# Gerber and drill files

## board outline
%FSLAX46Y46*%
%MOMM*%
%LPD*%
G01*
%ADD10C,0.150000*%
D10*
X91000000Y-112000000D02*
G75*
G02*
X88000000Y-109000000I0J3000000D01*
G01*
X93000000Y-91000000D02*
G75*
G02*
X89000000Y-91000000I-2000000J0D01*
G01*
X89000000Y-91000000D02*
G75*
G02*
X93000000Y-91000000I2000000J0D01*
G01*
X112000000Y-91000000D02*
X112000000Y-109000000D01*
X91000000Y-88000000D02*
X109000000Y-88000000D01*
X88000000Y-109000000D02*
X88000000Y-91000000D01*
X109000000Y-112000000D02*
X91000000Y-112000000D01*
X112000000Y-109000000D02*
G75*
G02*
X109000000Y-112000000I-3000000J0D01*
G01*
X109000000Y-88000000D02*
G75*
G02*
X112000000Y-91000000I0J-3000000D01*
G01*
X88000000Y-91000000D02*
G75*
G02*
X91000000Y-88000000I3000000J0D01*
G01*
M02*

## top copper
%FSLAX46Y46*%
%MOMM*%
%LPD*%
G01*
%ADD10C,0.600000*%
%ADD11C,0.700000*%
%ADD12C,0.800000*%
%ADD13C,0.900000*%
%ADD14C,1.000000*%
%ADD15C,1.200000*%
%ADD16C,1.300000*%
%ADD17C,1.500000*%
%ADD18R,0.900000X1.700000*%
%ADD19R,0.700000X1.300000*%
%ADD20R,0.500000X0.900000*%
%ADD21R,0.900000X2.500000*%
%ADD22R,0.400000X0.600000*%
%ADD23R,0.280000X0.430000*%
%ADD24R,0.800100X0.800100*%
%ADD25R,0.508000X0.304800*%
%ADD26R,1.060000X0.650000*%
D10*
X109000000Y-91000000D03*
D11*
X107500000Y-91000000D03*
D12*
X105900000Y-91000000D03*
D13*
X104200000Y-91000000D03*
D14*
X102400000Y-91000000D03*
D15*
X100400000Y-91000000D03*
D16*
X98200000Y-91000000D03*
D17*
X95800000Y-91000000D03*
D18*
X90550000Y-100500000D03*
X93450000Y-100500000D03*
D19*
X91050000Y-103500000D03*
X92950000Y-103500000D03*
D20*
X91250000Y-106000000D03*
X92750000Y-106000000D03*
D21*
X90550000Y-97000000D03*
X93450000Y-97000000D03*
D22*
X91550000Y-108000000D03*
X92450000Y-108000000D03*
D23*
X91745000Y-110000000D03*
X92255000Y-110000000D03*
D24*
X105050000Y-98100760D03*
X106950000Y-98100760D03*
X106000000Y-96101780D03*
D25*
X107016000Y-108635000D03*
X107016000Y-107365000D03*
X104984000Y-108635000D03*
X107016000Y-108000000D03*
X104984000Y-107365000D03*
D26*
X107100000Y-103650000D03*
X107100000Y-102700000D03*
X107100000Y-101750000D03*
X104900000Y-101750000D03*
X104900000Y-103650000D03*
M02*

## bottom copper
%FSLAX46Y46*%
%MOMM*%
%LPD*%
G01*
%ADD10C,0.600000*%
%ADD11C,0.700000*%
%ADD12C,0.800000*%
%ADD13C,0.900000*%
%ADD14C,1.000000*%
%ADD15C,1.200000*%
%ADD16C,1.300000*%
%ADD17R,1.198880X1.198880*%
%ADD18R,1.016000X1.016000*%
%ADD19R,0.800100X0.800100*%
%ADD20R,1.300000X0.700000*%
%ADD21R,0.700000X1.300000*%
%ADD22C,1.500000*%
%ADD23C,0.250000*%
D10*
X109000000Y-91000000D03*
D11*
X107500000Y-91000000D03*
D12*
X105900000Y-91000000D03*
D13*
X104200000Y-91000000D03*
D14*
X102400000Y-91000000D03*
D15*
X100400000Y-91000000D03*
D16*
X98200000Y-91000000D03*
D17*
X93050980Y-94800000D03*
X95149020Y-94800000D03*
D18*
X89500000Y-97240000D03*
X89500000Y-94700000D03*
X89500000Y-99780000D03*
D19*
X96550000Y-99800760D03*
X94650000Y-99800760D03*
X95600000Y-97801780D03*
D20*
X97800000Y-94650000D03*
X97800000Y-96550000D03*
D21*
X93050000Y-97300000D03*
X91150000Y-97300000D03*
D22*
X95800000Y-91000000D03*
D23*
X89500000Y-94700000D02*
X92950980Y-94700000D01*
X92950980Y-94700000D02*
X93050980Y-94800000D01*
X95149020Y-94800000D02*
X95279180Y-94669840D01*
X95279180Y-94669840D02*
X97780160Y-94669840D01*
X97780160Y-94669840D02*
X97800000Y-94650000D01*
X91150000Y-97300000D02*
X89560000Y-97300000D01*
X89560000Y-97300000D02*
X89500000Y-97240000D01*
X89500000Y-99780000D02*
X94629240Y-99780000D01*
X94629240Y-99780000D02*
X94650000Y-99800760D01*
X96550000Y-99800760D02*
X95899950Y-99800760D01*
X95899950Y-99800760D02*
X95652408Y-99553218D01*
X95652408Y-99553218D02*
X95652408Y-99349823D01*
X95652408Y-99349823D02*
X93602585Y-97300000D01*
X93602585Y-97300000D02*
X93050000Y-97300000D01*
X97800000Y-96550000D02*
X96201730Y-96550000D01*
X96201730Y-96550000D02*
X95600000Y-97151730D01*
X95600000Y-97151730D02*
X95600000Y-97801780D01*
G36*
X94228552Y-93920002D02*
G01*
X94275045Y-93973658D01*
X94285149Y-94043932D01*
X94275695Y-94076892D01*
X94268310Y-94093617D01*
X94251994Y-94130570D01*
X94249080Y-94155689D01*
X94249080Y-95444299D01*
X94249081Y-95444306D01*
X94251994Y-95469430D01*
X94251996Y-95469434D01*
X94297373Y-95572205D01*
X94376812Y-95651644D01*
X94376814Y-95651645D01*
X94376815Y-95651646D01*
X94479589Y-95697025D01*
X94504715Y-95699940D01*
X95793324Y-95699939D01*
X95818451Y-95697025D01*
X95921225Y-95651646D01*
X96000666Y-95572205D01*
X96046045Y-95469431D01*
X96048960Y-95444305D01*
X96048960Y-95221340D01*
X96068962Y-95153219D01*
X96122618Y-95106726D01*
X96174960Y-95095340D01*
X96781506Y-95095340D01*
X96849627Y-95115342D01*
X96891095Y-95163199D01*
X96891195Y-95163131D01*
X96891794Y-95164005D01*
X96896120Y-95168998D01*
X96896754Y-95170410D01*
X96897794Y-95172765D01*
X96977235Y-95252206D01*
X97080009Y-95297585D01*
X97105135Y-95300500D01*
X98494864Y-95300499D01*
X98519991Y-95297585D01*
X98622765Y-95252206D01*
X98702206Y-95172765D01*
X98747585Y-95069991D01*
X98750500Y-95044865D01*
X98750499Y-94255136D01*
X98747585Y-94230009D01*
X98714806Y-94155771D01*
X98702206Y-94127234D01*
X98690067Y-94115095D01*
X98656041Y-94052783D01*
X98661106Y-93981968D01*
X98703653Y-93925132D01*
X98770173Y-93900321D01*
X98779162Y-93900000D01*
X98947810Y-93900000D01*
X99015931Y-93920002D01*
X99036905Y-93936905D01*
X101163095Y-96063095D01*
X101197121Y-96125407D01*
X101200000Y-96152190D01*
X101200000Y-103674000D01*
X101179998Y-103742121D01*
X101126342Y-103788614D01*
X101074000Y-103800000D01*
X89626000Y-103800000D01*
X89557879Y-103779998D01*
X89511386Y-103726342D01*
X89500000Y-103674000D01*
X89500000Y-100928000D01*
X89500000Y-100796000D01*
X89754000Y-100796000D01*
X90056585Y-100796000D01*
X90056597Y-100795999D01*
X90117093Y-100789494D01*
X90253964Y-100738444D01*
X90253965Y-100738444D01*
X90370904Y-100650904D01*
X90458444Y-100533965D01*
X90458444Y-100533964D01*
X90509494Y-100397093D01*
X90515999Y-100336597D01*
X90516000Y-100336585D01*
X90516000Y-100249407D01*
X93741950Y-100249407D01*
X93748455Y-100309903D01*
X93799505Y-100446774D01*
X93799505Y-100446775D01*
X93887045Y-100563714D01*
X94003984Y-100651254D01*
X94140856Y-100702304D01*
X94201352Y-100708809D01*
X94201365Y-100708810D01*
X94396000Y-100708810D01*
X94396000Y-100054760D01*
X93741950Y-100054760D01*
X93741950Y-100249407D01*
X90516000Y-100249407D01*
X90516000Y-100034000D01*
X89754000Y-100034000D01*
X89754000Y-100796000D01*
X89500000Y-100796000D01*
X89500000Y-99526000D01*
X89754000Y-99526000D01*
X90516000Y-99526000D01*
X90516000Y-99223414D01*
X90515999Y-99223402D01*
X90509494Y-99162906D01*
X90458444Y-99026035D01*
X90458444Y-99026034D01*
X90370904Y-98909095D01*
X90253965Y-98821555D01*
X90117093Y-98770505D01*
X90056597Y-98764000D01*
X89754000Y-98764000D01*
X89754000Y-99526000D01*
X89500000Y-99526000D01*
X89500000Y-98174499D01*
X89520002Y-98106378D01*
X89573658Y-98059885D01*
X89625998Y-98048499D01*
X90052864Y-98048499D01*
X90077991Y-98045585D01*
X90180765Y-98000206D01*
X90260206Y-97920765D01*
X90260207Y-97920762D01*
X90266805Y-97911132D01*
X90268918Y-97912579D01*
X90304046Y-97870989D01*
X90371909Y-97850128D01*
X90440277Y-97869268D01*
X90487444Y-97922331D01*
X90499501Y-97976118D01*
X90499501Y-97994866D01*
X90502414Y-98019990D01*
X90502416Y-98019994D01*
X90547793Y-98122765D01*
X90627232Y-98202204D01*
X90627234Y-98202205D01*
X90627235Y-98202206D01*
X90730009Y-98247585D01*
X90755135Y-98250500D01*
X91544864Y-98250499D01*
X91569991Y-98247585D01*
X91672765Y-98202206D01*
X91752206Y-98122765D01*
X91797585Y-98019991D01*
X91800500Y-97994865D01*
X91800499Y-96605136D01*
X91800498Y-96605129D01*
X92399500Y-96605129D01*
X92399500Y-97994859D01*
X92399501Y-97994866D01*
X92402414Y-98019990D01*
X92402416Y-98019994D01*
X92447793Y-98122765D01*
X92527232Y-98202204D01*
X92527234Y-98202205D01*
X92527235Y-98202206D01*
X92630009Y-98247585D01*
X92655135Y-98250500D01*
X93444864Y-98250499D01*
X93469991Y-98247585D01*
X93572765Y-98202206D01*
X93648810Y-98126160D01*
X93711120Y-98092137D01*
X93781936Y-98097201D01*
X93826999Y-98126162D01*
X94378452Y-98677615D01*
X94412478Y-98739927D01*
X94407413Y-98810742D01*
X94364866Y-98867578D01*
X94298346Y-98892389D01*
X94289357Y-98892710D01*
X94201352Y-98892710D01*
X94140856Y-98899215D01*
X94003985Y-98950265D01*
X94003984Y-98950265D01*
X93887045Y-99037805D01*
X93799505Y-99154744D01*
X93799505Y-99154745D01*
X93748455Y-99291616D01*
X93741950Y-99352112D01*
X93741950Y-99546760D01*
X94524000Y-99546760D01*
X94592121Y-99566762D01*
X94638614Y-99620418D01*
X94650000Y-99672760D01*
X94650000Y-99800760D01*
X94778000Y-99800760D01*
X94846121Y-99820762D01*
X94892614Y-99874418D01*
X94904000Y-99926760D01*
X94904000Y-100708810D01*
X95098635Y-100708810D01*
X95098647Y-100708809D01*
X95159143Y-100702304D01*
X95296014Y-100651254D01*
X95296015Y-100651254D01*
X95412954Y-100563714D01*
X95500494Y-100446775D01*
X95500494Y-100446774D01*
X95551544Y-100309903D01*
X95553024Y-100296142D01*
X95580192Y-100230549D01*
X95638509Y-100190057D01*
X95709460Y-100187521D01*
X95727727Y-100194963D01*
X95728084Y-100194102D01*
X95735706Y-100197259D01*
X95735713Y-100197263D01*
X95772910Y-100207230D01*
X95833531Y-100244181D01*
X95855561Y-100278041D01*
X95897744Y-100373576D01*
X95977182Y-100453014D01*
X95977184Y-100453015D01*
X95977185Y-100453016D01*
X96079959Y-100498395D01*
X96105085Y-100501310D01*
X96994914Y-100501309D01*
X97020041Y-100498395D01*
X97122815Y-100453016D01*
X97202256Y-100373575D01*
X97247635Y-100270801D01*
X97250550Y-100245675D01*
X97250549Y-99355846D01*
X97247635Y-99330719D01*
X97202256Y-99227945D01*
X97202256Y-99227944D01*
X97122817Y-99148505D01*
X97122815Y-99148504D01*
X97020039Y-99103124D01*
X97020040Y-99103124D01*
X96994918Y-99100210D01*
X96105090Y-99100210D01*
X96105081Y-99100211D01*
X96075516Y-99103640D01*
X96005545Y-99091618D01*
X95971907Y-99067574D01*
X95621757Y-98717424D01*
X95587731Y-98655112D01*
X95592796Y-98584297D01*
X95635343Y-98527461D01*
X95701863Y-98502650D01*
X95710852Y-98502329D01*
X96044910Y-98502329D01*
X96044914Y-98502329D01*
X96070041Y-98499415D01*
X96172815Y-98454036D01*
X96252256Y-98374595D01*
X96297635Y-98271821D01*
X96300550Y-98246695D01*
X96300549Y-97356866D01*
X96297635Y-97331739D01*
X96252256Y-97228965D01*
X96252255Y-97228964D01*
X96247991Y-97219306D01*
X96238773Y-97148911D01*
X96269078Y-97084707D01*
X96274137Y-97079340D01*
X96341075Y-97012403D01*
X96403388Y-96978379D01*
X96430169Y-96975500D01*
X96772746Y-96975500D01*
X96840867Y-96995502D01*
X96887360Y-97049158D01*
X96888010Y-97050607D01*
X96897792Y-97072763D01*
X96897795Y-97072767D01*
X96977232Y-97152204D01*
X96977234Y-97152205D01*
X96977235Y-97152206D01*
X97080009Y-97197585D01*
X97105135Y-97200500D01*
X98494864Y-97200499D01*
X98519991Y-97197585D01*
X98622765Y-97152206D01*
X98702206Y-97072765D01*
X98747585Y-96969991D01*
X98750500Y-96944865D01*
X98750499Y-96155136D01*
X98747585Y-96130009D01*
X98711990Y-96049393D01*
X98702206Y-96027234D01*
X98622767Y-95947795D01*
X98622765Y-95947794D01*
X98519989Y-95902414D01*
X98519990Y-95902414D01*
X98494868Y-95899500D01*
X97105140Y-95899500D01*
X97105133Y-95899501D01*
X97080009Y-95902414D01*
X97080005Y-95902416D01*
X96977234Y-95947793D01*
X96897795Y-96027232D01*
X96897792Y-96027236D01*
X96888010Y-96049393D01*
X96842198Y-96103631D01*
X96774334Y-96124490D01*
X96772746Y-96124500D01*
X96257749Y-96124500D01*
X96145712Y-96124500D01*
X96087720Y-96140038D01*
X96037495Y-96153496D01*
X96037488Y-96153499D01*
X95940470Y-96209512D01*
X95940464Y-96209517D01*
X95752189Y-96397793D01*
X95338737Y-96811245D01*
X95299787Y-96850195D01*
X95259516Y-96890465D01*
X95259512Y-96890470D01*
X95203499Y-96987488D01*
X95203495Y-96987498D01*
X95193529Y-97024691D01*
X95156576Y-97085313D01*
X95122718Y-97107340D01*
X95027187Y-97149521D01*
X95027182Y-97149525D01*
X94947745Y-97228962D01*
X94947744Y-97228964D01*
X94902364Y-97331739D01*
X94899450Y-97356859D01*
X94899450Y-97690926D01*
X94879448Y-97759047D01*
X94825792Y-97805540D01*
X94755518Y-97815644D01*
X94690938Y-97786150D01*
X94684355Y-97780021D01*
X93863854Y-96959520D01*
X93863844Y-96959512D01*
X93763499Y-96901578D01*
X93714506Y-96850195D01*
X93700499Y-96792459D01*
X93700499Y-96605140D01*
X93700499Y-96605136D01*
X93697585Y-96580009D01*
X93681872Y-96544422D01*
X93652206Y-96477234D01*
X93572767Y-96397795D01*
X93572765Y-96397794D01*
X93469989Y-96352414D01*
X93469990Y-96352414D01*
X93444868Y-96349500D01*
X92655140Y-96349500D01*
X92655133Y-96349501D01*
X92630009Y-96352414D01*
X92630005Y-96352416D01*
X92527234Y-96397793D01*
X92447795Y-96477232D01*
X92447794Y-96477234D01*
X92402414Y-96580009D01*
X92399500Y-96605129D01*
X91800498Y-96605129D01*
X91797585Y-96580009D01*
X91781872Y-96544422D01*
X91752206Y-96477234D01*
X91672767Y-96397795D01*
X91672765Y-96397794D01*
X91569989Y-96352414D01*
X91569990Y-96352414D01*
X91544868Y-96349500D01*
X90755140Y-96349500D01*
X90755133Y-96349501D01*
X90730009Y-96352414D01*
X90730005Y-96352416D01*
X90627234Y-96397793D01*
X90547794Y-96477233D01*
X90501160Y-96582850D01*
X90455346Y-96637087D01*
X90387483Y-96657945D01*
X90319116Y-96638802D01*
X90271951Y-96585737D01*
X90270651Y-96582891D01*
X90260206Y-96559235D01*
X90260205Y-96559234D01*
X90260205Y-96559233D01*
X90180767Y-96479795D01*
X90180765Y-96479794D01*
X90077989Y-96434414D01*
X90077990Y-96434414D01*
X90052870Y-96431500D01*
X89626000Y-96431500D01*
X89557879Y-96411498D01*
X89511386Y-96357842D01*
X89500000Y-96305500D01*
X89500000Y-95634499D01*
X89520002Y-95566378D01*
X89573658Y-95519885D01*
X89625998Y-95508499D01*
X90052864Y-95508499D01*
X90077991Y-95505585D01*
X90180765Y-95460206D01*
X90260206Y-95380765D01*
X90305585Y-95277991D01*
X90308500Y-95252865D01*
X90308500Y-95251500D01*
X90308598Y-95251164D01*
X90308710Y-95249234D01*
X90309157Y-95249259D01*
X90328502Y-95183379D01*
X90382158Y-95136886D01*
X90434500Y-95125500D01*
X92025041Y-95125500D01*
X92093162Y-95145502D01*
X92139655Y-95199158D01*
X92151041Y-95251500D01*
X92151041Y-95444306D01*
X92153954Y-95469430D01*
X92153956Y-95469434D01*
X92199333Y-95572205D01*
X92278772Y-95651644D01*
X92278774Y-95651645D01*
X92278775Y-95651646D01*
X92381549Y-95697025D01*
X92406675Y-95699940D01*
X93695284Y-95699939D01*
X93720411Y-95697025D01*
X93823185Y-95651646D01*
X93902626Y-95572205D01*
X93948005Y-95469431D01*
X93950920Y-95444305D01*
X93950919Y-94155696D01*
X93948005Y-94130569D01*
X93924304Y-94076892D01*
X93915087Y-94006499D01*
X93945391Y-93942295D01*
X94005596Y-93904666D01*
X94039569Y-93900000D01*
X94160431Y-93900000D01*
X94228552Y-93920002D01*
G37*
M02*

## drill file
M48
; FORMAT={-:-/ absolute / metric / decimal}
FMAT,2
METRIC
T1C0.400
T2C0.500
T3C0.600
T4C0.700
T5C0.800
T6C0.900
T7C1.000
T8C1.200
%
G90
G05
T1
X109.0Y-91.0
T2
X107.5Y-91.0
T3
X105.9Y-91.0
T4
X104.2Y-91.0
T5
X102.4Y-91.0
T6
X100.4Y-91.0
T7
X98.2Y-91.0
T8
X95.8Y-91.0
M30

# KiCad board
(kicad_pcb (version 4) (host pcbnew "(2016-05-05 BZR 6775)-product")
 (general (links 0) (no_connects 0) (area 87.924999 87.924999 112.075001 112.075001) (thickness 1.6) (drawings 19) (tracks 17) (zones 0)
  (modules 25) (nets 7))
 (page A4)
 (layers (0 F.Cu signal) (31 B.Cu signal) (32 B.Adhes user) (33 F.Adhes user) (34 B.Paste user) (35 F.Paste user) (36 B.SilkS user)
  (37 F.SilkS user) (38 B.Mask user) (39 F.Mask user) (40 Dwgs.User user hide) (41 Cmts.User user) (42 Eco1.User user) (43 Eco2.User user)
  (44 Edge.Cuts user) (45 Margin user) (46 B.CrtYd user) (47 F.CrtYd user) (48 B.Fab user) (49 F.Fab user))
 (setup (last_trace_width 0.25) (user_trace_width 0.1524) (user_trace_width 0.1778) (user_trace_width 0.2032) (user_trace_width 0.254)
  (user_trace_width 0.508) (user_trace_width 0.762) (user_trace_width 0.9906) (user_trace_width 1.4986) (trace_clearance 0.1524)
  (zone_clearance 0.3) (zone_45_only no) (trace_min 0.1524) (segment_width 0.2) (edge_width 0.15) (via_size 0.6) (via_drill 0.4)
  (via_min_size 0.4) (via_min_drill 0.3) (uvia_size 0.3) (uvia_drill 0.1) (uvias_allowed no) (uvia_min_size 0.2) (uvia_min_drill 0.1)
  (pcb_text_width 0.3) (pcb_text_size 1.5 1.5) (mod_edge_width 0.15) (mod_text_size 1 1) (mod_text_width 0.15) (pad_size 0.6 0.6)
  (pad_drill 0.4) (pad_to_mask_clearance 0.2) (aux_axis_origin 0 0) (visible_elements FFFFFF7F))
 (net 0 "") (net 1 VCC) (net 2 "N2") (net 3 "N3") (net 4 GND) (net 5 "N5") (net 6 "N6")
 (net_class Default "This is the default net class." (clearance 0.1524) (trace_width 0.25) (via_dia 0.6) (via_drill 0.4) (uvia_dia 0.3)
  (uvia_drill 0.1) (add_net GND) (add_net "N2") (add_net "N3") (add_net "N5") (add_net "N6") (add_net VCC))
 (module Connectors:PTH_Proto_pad (layer F.Cu) (at 109 91)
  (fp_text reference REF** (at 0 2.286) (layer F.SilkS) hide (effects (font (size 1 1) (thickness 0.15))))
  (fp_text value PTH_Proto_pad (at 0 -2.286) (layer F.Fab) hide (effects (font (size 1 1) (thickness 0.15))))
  (pad 1 thru_hole circle (at 0 0) (size 0.6 0.6) (drill 0.4) (layers *.Cu *.Mask F.SilkS)))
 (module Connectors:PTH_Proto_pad (layer F.Cu) (at 107.5 91)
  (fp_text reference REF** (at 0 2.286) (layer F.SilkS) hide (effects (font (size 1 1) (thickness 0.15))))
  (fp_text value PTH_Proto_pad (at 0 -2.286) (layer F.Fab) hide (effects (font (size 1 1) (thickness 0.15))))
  (pad 1 thru_hole circle (at 0 0) (size 0.7 0.7) (drill 0.5) (layers *.Cu *.Mask F.SilkS)))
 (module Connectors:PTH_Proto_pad (layer F.Cu) (at 105.9 91)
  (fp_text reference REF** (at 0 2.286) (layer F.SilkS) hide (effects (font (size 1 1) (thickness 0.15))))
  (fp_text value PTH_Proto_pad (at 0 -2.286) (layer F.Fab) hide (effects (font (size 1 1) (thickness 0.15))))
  (pad 1 thru_hole circle (at 0 0) (size 0.8 0.8) (drill 0.6) (layers *.Cu *.Mask F.SilkS)))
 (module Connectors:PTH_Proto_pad (layer F.Cu) (at 104.2 91)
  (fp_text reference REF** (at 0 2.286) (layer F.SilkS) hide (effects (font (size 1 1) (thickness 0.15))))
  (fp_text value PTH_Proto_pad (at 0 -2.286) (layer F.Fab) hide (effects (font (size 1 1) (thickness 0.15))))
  (pad 1 thru_hole circle (at 0 0) (size 0.9 0.9) (drill 0.7) (layers *.Cu *.Mask F.SilkS)))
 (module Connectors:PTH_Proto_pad (layer F.Cu) (at 102.4 91)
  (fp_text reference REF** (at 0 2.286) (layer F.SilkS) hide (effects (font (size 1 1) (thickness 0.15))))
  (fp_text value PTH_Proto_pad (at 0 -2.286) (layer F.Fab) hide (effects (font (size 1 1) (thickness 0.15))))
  (pad 1 thru_hole circle (at 0 0) (size 1 1) (drill 0.8) (layers *.Cu *.Mask F.SilkS)))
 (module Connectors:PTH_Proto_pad (layer F.Cu) (at 100.4 91)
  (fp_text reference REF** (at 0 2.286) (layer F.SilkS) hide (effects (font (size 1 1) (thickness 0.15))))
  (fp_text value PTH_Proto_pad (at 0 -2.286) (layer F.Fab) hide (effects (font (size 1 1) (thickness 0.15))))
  (pad 1 thru_hole circle (at 0 0) (size 1.2 1.2) (drill 0.9) (layers *.Cu *.Mask F.SilkS)))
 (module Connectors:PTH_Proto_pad (layer F.Cu) (at 98.2 91)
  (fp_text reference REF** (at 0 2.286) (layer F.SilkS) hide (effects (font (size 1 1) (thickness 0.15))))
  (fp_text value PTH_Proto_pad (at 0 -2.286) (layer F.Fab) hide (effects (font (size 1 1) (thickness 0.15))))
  (pad 1 thru_hole circle (at 0 0) (size 1.3 1.3) (drill 1) (layers *.Cu *.Mask F.SilkS)))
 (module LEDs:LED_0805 (layer B.Cu) (at 94.1 94.8 180)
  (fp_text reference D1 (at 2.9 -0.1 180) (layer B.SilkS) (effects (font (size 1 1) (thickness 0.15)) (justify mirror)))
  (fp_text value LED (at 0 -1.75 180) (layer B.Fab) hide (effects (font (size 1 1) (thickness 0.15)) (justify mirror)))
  (pad 2 smd rect (at 1.04902 0) (size 1.19888 1.19888) (layers B.Cu B.Paste B.Mask) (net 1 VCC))
  (pad 1 smd rect (at -1.04902 0) (size 1.19888 1.19888) (layers B.Cu B.Paste B.Mask) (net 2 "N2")))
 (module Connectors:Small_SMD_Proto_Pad (layer B.Cu) (at 89.5 97.24)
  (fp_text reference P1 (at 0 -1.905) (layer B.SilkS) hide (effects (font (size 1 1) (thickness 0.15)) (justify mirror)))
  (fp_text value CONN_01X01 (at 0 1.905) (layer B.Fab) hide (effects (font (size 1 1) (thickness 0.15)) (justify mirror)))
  (pad 1 smd rect (at 0 0) (size 1.016 1.016) (layers B.Cu B.Paste B.Mask) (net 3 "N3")))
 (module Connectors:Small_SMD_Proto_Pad (layer B.Cu) (at 89.5 94.7)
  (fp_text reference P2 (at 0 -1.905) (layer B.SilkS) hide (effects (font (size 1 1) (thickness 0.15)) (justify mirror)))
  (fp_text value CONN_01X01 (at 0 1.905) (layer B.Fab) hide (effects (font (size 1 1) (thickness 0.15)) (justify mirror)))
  (pad 1 smd rect (at 0 0) (size 1.016 1.016) (layers B.Cu B.Paste B.Mask) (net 1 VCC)))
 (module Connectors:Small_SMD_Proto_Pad (layer B.Cu) (at 89.5 99.78)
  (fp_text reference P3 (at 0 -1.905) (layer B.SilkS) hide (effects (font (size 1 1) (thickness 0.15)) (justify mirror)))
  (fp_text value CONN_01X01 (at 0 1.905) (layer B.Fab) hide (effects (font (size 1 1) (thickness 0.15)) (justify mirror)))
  (pad 1 smd rect (at 0 0) (size 1.016 1.016) (layers B.Cu B.Paste B.Mask) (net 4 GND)))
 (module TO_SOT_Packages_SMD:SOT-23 (layer B.Cu) (at 95.6 98.8 180)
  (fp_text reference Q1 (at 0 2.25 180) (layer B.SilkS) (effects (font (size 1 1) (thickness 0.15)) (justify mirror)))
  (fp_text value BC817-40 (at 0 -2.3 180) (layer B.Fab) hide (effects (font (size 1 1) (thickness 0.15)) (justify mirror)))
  (pad 1 smd rect (at -0.95 -1.00076 180) (size 0.8001 0.8001) (layers B.Cu B.Paste B.Mask) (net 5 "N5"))
  (pad 2 smd rect (at 0.95 -1.00076 180) (size 0.8001 0.8001) (layers B.Cu B.Paste B.Mask) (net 4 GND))
  (pad 3 smd rect (at 0 0.99822 180) (size 0.8001 0.8001) (layers B.Cu B.Paste B.Mask) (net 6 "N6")))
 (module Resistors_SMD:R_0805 (layer B.Cu) (at 97.8 95.6 270)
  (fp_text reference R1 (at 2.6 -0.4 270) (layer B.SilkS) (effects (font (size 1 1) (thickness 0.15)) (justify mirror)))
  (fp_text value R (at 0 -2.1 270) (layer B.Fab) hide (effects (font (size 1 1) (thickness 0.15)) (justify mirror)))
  (pad 1 smd rect (at -0.95 0 270) (size 0.7 1.3) (layers B.Cu B.Paste B.Mask) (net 2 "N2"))
  (pad 2 smd rect (at 0.95 0 270) (size 0.7 1.3) (layers B.Cu B.Paste B.Mask) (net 6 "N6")))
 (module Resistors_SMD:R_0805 (layer B.Cu) (at 92.1 97.3 180)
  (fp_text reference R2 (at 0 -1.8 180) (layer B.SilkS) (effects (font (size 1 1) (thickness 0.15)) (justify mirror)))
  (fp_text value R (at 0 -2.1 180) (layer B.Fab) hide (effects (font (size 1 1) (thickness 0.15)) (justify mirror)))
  (pad 1 smd rect (at -0.95 0 180) (size 0.7 1.3) (layers B.Cu B.Paste B.Mask) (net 5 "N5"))
  (pad 2 smd rect (at 0.95 0 180) (size 0.7 1.3) (layers B.Cu B.Paste B.Mask) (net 3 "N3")))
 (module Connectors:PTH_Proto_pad (layer F.Cu) (at 95.8 91)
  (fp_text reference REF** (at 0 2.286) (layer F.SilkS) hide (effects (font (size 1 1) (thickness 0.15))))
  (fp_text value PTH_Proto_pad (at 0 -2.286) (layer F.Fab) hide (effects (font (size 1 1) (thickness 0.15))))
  (pad 1 thru_hole circle (at 0 0) (size 1.5 1.5) (drill 1.2) (layers *.Cu *.Mask F.SilkS)))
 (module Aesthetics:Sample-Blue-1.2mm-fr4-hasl (layer B.Cu) (at 100 102.6 180)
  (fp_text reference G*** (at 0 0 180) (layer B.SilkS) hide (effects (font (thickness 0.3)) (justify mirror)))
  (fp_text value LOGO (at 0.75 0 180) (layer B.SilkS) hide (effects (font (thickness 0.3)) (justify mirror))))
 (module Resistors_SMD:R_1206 (layer F.Cu) (at 92 100.5)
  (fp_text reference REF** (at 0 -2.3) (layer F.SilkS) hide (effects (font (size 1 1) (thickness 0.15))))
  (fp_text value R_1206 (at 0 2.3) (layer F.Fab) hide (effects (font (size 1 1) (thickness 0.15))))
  (pad 1 smd rect (at -1.45 0) (size 0.9 1.7) (layers F.Cu F.Paste F.Mask))
  (pad 2 smd rect (at 1.45 0) (size 0.9 1.7) (layers F.Cu F.Paste F.Mask)))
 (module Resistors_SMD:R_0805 (layer F.Cu) (at 92 103.5)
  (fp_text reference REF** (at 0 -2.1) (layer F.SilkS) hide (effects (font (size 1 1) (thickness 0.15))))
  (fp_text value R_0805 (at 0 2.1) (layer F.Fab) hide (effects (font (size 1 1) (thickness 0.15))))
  (pad 1 smd rect (at -0.95 0) (size 0.7 1.3) (layers F.Cu F.Paste F.Mask))
  (pad 2 smd rect (at 0.95 0) (size 0.7 1.3) (layers F.Cu F.Paste F.Mask)))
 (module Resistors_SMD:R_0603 (layer F.Cu) (at 92 106)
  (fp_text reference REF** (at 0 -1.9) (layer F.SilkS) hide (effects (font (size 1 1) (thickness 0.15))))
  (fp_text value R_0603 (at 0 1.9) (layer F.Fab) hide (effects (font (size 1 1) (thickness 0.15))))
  (pad 1 smd rect (at -0.75 0) (size 0.5 0.9) (layers F.Cu F.Paste F.Mask))
  (pad 2 smd rect (at 0.75 0) (size 0.5 0.9) (layers F.Cu F.Paste F.Mask)))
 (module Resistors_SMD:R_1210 (layer F.Cu) (at 92 97)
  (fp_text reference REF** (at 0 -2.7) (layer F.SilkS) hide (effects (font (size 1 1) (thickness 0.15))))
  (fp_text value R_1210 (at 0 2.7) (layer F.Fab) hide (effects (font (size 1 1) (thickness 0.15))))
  (pad 1 smd rect (at -1.45 0) (size 0.9 2.5) (layers F.Cu F.Paste F.Mask))
  (pad 2 smd rect (at 1.45 0) (size 0.9 2.5) (layers F.Cu F.Paste F.Mask)))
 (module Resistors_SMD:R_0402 (layer F.Cu) (at 92 108)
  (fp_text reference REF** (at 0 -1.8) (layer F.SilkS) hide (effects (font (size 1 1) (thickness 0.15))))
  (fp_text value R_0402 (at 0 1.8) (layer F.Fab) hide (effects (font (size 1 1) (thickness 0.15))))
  (pad 1 smd rect (at -0.45 0) (size 0.4 0.6) (layers F.Cu F.Paste F.Mask))
  (pad 2 smd rect (at 0.45 0) (size 0.4 0.6) (layers F.Cu F.Paste F.Mask)))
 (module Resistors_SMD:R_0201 (layer F.Cu) (at 92 110)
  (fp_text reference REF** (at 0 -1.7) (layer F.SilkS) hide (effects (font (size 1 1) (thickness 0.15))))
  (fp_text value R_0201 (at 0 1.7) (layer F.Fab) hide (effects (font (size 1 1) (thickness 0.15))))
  (pad 1 smd rect (at -0.255 0) (size 0.28 0.43) (layers F.Cu F.Paste F.Mask))
  (pad 2 smd rect (at 0.255 0) (size 0.28 0.43) (layers F.Cu F.Paste F.Mask)))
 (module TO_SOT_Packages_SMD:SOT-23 (layer F.Cu) (at 106 97.1)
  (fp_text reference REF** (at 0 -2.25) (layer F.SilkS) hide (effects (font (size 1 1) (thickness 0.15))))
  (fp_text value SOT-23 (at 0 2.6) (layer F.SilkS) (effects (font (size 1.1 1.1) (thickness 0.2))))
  (pad 1 smd rect (at -0.95 1.00076) (size 0.8001 0.8001) (layers F.Cu F.Paste F.Mask))
  (pad 2 smd rect (at 0.95 1.00076) (size 0.8001 0.8001) (layers F.Cu F.Paste F.Mask))
  (pad 3 smd rect (at 0 -0.99822) (size 0.8001 0.8001) (layers F.Cu F.Paste F.Mask)))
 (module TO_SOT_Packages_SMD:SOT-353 (layer F.Cu) (at 106 108 180)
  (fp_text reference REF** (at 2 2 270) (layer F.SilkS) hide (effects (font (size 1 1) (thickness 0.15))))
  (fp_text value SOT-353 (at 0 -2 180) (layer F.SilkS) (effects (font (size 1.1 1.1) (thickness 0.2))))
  (pad 1 smd rect (at -1.016 -0.635 180) (size 0.508 0.3048) (layers F.Cu F.Paste F.Mask))
  (pad 3 smd rect (at -1.016 0.635 180) (size 0.508 0.3048) (layers F.Cu F.Paste F.Mask))
  (pad 5 smd rect (at 1.016 -0.635 180) (size 0.508 0.3048) (layers F.Cu F.Paste F.Mask))
  (pad 2 smd rect (at -1.016 0 180) (size 0.508 0.3048) (layers F.Cu F.Paste F.Mask))
  (pad 4 smd rect (at 1.016 0.635 180) (size 0.508 0.3048) (layers F.Cu F.Paste F.Mask)))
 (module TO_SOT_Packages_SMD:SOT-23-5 (layer F.Cu) (at 106 102.7 180)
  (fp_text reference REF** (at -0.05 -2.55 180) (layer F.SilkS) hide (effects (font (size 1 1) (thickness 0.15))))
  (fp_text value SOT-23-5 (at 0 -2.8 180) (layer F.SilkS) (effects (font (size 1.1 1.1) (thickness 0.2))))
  (pad 1 smd rect (at -1.1 -0.95 180) (size 1.06 0.65) (layers F.Cu F.Paste F.Mask))
  (pad 2 smd rect (at -1.1 0 180) (size 1.06 0.65) (layers F.Cu F.Paste F.Mask))
  (pad 3 smd rect (at -1.1 0.95 180) (size 1.06 0.65) (layers F.Cu F.Paste F.Mask))
  (pad 4 smd rect (at 1.1 0.95 180) (size 1.06 0.65) (layers F.Cu F.Paste F.Mask))
  (pad 5 smd rect (at 1.1 -0.95 180) (size 1.06 0.65) (layers F.Cu F.Paste F.Mask)))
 (gr_arc (start 91 109) (end 91 112) (angle 90) (layer Edge.Cuts) (width 0.15))
 (gr_circle (center 91 91) (end 93 91) (layer Edge.Cuts) (width 0.15))
 (gr_line (start 112 91) (end 112 109) (layer Edge.Cuts) (width 0.15))
 (gr_line (start 91 88) (end 109 88) (layer Edge.Cuts) (width 0.15))
 (gr_line (start 88 109) (end 88 91) (layer Edge.Cuts) (width 0.15))
 (gr_line (start 109 112) (end 91 112) (layer Edge.Cuts) (width 0.15))
 (gr_arc (start 109 109) (end 112 109) (angle 90) (layer Edge.Cuts) (width 0.15))
 (gr_arc (start 109 91) (end 109 88) (angle 90) (layer Edge.Cuts) (width 0.15))
 (gr_arc (start 91 91) (end 88 91) (angle 90) (layer Edge.Cuts) (width 0.15))
 (segment (start 89.5 94.7) (end 92.95098 94.7) (width 0.25) (layer B.Cu) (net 1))
 (segment (start 92.95098 94.7) (end 93.05098 94.8) (width 0.25) (layer B.Cu) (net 1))
 (segment (start 95.14902 94.8) (end 95.27918 94.66984) (width 0.25) (layer B.Cu) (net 2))
 (segment (start 95.27918 94.66984) (end 97.78016 94.66984) (width 0.25) (layer B.Cu) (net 2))
 (segment (start 97.78016 94.66984) (end 97.8 94.65) (width 0.25) (layer B.Cu) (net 2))
 (segment (start 91.15 97.3) (end 89.56 97.3) (width 0.25) (layer B.Cu) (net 3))
 (segment (start 89.56 97.3) (end 89.5 97.24) (width 0.25) (layer B.Cu) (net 3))
 (segment (start 89.5 99.78) (end 94.62924 99.78) (width 0.25) (layer B.Cu) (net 4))
 (segment (start 94.62924 99.78) (end 94.65 99.80076) (width 0.25) (layer B.Cu) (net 4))
 (segment (start 96.55 99.80076) (end 95.89995 99.80076) (width 0.25) (layer B.Cu) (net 5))
 (segment (start 95.89995 99.80076) (end 95.652408 99.553218) (width 0.25) (layer B.Cu) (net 5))
 (segment (start 95.652408 99.553218) (end 95.652408 99.349823) (width 0.25) (layer B.Cu) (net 5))
 (segment (start 95.652408 99.349823) (end 93.602585 97.3) (width 0.25) (layer B.Cu) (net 5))
 (segment (start 93.602585 97.3) (end 93.05 97.3) (width 0.25) (layer B.Cu) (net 5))
 (segment (start 97.8 96.55) (end 96.20173 96.55) (width 0.25) (layer B.Cu) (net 6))
 (segment (start 96.20173 96.55) (end 95.6 97.15173) (width 0.25) (layer B.Cu) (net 6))
 (segment (start 95.6 97.15173) (end 95.6 97.80178) (width 0.25) (layer B.Cu) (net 6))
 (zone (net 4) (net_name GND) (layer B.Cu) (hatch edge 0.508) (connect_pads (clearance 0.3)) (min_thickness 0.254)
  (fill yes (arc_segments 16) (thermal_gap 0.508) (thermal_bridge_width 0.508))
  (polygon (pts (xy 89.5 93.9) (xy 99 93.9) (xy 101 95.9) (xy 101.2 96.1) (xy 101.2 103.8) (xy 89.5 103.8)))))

